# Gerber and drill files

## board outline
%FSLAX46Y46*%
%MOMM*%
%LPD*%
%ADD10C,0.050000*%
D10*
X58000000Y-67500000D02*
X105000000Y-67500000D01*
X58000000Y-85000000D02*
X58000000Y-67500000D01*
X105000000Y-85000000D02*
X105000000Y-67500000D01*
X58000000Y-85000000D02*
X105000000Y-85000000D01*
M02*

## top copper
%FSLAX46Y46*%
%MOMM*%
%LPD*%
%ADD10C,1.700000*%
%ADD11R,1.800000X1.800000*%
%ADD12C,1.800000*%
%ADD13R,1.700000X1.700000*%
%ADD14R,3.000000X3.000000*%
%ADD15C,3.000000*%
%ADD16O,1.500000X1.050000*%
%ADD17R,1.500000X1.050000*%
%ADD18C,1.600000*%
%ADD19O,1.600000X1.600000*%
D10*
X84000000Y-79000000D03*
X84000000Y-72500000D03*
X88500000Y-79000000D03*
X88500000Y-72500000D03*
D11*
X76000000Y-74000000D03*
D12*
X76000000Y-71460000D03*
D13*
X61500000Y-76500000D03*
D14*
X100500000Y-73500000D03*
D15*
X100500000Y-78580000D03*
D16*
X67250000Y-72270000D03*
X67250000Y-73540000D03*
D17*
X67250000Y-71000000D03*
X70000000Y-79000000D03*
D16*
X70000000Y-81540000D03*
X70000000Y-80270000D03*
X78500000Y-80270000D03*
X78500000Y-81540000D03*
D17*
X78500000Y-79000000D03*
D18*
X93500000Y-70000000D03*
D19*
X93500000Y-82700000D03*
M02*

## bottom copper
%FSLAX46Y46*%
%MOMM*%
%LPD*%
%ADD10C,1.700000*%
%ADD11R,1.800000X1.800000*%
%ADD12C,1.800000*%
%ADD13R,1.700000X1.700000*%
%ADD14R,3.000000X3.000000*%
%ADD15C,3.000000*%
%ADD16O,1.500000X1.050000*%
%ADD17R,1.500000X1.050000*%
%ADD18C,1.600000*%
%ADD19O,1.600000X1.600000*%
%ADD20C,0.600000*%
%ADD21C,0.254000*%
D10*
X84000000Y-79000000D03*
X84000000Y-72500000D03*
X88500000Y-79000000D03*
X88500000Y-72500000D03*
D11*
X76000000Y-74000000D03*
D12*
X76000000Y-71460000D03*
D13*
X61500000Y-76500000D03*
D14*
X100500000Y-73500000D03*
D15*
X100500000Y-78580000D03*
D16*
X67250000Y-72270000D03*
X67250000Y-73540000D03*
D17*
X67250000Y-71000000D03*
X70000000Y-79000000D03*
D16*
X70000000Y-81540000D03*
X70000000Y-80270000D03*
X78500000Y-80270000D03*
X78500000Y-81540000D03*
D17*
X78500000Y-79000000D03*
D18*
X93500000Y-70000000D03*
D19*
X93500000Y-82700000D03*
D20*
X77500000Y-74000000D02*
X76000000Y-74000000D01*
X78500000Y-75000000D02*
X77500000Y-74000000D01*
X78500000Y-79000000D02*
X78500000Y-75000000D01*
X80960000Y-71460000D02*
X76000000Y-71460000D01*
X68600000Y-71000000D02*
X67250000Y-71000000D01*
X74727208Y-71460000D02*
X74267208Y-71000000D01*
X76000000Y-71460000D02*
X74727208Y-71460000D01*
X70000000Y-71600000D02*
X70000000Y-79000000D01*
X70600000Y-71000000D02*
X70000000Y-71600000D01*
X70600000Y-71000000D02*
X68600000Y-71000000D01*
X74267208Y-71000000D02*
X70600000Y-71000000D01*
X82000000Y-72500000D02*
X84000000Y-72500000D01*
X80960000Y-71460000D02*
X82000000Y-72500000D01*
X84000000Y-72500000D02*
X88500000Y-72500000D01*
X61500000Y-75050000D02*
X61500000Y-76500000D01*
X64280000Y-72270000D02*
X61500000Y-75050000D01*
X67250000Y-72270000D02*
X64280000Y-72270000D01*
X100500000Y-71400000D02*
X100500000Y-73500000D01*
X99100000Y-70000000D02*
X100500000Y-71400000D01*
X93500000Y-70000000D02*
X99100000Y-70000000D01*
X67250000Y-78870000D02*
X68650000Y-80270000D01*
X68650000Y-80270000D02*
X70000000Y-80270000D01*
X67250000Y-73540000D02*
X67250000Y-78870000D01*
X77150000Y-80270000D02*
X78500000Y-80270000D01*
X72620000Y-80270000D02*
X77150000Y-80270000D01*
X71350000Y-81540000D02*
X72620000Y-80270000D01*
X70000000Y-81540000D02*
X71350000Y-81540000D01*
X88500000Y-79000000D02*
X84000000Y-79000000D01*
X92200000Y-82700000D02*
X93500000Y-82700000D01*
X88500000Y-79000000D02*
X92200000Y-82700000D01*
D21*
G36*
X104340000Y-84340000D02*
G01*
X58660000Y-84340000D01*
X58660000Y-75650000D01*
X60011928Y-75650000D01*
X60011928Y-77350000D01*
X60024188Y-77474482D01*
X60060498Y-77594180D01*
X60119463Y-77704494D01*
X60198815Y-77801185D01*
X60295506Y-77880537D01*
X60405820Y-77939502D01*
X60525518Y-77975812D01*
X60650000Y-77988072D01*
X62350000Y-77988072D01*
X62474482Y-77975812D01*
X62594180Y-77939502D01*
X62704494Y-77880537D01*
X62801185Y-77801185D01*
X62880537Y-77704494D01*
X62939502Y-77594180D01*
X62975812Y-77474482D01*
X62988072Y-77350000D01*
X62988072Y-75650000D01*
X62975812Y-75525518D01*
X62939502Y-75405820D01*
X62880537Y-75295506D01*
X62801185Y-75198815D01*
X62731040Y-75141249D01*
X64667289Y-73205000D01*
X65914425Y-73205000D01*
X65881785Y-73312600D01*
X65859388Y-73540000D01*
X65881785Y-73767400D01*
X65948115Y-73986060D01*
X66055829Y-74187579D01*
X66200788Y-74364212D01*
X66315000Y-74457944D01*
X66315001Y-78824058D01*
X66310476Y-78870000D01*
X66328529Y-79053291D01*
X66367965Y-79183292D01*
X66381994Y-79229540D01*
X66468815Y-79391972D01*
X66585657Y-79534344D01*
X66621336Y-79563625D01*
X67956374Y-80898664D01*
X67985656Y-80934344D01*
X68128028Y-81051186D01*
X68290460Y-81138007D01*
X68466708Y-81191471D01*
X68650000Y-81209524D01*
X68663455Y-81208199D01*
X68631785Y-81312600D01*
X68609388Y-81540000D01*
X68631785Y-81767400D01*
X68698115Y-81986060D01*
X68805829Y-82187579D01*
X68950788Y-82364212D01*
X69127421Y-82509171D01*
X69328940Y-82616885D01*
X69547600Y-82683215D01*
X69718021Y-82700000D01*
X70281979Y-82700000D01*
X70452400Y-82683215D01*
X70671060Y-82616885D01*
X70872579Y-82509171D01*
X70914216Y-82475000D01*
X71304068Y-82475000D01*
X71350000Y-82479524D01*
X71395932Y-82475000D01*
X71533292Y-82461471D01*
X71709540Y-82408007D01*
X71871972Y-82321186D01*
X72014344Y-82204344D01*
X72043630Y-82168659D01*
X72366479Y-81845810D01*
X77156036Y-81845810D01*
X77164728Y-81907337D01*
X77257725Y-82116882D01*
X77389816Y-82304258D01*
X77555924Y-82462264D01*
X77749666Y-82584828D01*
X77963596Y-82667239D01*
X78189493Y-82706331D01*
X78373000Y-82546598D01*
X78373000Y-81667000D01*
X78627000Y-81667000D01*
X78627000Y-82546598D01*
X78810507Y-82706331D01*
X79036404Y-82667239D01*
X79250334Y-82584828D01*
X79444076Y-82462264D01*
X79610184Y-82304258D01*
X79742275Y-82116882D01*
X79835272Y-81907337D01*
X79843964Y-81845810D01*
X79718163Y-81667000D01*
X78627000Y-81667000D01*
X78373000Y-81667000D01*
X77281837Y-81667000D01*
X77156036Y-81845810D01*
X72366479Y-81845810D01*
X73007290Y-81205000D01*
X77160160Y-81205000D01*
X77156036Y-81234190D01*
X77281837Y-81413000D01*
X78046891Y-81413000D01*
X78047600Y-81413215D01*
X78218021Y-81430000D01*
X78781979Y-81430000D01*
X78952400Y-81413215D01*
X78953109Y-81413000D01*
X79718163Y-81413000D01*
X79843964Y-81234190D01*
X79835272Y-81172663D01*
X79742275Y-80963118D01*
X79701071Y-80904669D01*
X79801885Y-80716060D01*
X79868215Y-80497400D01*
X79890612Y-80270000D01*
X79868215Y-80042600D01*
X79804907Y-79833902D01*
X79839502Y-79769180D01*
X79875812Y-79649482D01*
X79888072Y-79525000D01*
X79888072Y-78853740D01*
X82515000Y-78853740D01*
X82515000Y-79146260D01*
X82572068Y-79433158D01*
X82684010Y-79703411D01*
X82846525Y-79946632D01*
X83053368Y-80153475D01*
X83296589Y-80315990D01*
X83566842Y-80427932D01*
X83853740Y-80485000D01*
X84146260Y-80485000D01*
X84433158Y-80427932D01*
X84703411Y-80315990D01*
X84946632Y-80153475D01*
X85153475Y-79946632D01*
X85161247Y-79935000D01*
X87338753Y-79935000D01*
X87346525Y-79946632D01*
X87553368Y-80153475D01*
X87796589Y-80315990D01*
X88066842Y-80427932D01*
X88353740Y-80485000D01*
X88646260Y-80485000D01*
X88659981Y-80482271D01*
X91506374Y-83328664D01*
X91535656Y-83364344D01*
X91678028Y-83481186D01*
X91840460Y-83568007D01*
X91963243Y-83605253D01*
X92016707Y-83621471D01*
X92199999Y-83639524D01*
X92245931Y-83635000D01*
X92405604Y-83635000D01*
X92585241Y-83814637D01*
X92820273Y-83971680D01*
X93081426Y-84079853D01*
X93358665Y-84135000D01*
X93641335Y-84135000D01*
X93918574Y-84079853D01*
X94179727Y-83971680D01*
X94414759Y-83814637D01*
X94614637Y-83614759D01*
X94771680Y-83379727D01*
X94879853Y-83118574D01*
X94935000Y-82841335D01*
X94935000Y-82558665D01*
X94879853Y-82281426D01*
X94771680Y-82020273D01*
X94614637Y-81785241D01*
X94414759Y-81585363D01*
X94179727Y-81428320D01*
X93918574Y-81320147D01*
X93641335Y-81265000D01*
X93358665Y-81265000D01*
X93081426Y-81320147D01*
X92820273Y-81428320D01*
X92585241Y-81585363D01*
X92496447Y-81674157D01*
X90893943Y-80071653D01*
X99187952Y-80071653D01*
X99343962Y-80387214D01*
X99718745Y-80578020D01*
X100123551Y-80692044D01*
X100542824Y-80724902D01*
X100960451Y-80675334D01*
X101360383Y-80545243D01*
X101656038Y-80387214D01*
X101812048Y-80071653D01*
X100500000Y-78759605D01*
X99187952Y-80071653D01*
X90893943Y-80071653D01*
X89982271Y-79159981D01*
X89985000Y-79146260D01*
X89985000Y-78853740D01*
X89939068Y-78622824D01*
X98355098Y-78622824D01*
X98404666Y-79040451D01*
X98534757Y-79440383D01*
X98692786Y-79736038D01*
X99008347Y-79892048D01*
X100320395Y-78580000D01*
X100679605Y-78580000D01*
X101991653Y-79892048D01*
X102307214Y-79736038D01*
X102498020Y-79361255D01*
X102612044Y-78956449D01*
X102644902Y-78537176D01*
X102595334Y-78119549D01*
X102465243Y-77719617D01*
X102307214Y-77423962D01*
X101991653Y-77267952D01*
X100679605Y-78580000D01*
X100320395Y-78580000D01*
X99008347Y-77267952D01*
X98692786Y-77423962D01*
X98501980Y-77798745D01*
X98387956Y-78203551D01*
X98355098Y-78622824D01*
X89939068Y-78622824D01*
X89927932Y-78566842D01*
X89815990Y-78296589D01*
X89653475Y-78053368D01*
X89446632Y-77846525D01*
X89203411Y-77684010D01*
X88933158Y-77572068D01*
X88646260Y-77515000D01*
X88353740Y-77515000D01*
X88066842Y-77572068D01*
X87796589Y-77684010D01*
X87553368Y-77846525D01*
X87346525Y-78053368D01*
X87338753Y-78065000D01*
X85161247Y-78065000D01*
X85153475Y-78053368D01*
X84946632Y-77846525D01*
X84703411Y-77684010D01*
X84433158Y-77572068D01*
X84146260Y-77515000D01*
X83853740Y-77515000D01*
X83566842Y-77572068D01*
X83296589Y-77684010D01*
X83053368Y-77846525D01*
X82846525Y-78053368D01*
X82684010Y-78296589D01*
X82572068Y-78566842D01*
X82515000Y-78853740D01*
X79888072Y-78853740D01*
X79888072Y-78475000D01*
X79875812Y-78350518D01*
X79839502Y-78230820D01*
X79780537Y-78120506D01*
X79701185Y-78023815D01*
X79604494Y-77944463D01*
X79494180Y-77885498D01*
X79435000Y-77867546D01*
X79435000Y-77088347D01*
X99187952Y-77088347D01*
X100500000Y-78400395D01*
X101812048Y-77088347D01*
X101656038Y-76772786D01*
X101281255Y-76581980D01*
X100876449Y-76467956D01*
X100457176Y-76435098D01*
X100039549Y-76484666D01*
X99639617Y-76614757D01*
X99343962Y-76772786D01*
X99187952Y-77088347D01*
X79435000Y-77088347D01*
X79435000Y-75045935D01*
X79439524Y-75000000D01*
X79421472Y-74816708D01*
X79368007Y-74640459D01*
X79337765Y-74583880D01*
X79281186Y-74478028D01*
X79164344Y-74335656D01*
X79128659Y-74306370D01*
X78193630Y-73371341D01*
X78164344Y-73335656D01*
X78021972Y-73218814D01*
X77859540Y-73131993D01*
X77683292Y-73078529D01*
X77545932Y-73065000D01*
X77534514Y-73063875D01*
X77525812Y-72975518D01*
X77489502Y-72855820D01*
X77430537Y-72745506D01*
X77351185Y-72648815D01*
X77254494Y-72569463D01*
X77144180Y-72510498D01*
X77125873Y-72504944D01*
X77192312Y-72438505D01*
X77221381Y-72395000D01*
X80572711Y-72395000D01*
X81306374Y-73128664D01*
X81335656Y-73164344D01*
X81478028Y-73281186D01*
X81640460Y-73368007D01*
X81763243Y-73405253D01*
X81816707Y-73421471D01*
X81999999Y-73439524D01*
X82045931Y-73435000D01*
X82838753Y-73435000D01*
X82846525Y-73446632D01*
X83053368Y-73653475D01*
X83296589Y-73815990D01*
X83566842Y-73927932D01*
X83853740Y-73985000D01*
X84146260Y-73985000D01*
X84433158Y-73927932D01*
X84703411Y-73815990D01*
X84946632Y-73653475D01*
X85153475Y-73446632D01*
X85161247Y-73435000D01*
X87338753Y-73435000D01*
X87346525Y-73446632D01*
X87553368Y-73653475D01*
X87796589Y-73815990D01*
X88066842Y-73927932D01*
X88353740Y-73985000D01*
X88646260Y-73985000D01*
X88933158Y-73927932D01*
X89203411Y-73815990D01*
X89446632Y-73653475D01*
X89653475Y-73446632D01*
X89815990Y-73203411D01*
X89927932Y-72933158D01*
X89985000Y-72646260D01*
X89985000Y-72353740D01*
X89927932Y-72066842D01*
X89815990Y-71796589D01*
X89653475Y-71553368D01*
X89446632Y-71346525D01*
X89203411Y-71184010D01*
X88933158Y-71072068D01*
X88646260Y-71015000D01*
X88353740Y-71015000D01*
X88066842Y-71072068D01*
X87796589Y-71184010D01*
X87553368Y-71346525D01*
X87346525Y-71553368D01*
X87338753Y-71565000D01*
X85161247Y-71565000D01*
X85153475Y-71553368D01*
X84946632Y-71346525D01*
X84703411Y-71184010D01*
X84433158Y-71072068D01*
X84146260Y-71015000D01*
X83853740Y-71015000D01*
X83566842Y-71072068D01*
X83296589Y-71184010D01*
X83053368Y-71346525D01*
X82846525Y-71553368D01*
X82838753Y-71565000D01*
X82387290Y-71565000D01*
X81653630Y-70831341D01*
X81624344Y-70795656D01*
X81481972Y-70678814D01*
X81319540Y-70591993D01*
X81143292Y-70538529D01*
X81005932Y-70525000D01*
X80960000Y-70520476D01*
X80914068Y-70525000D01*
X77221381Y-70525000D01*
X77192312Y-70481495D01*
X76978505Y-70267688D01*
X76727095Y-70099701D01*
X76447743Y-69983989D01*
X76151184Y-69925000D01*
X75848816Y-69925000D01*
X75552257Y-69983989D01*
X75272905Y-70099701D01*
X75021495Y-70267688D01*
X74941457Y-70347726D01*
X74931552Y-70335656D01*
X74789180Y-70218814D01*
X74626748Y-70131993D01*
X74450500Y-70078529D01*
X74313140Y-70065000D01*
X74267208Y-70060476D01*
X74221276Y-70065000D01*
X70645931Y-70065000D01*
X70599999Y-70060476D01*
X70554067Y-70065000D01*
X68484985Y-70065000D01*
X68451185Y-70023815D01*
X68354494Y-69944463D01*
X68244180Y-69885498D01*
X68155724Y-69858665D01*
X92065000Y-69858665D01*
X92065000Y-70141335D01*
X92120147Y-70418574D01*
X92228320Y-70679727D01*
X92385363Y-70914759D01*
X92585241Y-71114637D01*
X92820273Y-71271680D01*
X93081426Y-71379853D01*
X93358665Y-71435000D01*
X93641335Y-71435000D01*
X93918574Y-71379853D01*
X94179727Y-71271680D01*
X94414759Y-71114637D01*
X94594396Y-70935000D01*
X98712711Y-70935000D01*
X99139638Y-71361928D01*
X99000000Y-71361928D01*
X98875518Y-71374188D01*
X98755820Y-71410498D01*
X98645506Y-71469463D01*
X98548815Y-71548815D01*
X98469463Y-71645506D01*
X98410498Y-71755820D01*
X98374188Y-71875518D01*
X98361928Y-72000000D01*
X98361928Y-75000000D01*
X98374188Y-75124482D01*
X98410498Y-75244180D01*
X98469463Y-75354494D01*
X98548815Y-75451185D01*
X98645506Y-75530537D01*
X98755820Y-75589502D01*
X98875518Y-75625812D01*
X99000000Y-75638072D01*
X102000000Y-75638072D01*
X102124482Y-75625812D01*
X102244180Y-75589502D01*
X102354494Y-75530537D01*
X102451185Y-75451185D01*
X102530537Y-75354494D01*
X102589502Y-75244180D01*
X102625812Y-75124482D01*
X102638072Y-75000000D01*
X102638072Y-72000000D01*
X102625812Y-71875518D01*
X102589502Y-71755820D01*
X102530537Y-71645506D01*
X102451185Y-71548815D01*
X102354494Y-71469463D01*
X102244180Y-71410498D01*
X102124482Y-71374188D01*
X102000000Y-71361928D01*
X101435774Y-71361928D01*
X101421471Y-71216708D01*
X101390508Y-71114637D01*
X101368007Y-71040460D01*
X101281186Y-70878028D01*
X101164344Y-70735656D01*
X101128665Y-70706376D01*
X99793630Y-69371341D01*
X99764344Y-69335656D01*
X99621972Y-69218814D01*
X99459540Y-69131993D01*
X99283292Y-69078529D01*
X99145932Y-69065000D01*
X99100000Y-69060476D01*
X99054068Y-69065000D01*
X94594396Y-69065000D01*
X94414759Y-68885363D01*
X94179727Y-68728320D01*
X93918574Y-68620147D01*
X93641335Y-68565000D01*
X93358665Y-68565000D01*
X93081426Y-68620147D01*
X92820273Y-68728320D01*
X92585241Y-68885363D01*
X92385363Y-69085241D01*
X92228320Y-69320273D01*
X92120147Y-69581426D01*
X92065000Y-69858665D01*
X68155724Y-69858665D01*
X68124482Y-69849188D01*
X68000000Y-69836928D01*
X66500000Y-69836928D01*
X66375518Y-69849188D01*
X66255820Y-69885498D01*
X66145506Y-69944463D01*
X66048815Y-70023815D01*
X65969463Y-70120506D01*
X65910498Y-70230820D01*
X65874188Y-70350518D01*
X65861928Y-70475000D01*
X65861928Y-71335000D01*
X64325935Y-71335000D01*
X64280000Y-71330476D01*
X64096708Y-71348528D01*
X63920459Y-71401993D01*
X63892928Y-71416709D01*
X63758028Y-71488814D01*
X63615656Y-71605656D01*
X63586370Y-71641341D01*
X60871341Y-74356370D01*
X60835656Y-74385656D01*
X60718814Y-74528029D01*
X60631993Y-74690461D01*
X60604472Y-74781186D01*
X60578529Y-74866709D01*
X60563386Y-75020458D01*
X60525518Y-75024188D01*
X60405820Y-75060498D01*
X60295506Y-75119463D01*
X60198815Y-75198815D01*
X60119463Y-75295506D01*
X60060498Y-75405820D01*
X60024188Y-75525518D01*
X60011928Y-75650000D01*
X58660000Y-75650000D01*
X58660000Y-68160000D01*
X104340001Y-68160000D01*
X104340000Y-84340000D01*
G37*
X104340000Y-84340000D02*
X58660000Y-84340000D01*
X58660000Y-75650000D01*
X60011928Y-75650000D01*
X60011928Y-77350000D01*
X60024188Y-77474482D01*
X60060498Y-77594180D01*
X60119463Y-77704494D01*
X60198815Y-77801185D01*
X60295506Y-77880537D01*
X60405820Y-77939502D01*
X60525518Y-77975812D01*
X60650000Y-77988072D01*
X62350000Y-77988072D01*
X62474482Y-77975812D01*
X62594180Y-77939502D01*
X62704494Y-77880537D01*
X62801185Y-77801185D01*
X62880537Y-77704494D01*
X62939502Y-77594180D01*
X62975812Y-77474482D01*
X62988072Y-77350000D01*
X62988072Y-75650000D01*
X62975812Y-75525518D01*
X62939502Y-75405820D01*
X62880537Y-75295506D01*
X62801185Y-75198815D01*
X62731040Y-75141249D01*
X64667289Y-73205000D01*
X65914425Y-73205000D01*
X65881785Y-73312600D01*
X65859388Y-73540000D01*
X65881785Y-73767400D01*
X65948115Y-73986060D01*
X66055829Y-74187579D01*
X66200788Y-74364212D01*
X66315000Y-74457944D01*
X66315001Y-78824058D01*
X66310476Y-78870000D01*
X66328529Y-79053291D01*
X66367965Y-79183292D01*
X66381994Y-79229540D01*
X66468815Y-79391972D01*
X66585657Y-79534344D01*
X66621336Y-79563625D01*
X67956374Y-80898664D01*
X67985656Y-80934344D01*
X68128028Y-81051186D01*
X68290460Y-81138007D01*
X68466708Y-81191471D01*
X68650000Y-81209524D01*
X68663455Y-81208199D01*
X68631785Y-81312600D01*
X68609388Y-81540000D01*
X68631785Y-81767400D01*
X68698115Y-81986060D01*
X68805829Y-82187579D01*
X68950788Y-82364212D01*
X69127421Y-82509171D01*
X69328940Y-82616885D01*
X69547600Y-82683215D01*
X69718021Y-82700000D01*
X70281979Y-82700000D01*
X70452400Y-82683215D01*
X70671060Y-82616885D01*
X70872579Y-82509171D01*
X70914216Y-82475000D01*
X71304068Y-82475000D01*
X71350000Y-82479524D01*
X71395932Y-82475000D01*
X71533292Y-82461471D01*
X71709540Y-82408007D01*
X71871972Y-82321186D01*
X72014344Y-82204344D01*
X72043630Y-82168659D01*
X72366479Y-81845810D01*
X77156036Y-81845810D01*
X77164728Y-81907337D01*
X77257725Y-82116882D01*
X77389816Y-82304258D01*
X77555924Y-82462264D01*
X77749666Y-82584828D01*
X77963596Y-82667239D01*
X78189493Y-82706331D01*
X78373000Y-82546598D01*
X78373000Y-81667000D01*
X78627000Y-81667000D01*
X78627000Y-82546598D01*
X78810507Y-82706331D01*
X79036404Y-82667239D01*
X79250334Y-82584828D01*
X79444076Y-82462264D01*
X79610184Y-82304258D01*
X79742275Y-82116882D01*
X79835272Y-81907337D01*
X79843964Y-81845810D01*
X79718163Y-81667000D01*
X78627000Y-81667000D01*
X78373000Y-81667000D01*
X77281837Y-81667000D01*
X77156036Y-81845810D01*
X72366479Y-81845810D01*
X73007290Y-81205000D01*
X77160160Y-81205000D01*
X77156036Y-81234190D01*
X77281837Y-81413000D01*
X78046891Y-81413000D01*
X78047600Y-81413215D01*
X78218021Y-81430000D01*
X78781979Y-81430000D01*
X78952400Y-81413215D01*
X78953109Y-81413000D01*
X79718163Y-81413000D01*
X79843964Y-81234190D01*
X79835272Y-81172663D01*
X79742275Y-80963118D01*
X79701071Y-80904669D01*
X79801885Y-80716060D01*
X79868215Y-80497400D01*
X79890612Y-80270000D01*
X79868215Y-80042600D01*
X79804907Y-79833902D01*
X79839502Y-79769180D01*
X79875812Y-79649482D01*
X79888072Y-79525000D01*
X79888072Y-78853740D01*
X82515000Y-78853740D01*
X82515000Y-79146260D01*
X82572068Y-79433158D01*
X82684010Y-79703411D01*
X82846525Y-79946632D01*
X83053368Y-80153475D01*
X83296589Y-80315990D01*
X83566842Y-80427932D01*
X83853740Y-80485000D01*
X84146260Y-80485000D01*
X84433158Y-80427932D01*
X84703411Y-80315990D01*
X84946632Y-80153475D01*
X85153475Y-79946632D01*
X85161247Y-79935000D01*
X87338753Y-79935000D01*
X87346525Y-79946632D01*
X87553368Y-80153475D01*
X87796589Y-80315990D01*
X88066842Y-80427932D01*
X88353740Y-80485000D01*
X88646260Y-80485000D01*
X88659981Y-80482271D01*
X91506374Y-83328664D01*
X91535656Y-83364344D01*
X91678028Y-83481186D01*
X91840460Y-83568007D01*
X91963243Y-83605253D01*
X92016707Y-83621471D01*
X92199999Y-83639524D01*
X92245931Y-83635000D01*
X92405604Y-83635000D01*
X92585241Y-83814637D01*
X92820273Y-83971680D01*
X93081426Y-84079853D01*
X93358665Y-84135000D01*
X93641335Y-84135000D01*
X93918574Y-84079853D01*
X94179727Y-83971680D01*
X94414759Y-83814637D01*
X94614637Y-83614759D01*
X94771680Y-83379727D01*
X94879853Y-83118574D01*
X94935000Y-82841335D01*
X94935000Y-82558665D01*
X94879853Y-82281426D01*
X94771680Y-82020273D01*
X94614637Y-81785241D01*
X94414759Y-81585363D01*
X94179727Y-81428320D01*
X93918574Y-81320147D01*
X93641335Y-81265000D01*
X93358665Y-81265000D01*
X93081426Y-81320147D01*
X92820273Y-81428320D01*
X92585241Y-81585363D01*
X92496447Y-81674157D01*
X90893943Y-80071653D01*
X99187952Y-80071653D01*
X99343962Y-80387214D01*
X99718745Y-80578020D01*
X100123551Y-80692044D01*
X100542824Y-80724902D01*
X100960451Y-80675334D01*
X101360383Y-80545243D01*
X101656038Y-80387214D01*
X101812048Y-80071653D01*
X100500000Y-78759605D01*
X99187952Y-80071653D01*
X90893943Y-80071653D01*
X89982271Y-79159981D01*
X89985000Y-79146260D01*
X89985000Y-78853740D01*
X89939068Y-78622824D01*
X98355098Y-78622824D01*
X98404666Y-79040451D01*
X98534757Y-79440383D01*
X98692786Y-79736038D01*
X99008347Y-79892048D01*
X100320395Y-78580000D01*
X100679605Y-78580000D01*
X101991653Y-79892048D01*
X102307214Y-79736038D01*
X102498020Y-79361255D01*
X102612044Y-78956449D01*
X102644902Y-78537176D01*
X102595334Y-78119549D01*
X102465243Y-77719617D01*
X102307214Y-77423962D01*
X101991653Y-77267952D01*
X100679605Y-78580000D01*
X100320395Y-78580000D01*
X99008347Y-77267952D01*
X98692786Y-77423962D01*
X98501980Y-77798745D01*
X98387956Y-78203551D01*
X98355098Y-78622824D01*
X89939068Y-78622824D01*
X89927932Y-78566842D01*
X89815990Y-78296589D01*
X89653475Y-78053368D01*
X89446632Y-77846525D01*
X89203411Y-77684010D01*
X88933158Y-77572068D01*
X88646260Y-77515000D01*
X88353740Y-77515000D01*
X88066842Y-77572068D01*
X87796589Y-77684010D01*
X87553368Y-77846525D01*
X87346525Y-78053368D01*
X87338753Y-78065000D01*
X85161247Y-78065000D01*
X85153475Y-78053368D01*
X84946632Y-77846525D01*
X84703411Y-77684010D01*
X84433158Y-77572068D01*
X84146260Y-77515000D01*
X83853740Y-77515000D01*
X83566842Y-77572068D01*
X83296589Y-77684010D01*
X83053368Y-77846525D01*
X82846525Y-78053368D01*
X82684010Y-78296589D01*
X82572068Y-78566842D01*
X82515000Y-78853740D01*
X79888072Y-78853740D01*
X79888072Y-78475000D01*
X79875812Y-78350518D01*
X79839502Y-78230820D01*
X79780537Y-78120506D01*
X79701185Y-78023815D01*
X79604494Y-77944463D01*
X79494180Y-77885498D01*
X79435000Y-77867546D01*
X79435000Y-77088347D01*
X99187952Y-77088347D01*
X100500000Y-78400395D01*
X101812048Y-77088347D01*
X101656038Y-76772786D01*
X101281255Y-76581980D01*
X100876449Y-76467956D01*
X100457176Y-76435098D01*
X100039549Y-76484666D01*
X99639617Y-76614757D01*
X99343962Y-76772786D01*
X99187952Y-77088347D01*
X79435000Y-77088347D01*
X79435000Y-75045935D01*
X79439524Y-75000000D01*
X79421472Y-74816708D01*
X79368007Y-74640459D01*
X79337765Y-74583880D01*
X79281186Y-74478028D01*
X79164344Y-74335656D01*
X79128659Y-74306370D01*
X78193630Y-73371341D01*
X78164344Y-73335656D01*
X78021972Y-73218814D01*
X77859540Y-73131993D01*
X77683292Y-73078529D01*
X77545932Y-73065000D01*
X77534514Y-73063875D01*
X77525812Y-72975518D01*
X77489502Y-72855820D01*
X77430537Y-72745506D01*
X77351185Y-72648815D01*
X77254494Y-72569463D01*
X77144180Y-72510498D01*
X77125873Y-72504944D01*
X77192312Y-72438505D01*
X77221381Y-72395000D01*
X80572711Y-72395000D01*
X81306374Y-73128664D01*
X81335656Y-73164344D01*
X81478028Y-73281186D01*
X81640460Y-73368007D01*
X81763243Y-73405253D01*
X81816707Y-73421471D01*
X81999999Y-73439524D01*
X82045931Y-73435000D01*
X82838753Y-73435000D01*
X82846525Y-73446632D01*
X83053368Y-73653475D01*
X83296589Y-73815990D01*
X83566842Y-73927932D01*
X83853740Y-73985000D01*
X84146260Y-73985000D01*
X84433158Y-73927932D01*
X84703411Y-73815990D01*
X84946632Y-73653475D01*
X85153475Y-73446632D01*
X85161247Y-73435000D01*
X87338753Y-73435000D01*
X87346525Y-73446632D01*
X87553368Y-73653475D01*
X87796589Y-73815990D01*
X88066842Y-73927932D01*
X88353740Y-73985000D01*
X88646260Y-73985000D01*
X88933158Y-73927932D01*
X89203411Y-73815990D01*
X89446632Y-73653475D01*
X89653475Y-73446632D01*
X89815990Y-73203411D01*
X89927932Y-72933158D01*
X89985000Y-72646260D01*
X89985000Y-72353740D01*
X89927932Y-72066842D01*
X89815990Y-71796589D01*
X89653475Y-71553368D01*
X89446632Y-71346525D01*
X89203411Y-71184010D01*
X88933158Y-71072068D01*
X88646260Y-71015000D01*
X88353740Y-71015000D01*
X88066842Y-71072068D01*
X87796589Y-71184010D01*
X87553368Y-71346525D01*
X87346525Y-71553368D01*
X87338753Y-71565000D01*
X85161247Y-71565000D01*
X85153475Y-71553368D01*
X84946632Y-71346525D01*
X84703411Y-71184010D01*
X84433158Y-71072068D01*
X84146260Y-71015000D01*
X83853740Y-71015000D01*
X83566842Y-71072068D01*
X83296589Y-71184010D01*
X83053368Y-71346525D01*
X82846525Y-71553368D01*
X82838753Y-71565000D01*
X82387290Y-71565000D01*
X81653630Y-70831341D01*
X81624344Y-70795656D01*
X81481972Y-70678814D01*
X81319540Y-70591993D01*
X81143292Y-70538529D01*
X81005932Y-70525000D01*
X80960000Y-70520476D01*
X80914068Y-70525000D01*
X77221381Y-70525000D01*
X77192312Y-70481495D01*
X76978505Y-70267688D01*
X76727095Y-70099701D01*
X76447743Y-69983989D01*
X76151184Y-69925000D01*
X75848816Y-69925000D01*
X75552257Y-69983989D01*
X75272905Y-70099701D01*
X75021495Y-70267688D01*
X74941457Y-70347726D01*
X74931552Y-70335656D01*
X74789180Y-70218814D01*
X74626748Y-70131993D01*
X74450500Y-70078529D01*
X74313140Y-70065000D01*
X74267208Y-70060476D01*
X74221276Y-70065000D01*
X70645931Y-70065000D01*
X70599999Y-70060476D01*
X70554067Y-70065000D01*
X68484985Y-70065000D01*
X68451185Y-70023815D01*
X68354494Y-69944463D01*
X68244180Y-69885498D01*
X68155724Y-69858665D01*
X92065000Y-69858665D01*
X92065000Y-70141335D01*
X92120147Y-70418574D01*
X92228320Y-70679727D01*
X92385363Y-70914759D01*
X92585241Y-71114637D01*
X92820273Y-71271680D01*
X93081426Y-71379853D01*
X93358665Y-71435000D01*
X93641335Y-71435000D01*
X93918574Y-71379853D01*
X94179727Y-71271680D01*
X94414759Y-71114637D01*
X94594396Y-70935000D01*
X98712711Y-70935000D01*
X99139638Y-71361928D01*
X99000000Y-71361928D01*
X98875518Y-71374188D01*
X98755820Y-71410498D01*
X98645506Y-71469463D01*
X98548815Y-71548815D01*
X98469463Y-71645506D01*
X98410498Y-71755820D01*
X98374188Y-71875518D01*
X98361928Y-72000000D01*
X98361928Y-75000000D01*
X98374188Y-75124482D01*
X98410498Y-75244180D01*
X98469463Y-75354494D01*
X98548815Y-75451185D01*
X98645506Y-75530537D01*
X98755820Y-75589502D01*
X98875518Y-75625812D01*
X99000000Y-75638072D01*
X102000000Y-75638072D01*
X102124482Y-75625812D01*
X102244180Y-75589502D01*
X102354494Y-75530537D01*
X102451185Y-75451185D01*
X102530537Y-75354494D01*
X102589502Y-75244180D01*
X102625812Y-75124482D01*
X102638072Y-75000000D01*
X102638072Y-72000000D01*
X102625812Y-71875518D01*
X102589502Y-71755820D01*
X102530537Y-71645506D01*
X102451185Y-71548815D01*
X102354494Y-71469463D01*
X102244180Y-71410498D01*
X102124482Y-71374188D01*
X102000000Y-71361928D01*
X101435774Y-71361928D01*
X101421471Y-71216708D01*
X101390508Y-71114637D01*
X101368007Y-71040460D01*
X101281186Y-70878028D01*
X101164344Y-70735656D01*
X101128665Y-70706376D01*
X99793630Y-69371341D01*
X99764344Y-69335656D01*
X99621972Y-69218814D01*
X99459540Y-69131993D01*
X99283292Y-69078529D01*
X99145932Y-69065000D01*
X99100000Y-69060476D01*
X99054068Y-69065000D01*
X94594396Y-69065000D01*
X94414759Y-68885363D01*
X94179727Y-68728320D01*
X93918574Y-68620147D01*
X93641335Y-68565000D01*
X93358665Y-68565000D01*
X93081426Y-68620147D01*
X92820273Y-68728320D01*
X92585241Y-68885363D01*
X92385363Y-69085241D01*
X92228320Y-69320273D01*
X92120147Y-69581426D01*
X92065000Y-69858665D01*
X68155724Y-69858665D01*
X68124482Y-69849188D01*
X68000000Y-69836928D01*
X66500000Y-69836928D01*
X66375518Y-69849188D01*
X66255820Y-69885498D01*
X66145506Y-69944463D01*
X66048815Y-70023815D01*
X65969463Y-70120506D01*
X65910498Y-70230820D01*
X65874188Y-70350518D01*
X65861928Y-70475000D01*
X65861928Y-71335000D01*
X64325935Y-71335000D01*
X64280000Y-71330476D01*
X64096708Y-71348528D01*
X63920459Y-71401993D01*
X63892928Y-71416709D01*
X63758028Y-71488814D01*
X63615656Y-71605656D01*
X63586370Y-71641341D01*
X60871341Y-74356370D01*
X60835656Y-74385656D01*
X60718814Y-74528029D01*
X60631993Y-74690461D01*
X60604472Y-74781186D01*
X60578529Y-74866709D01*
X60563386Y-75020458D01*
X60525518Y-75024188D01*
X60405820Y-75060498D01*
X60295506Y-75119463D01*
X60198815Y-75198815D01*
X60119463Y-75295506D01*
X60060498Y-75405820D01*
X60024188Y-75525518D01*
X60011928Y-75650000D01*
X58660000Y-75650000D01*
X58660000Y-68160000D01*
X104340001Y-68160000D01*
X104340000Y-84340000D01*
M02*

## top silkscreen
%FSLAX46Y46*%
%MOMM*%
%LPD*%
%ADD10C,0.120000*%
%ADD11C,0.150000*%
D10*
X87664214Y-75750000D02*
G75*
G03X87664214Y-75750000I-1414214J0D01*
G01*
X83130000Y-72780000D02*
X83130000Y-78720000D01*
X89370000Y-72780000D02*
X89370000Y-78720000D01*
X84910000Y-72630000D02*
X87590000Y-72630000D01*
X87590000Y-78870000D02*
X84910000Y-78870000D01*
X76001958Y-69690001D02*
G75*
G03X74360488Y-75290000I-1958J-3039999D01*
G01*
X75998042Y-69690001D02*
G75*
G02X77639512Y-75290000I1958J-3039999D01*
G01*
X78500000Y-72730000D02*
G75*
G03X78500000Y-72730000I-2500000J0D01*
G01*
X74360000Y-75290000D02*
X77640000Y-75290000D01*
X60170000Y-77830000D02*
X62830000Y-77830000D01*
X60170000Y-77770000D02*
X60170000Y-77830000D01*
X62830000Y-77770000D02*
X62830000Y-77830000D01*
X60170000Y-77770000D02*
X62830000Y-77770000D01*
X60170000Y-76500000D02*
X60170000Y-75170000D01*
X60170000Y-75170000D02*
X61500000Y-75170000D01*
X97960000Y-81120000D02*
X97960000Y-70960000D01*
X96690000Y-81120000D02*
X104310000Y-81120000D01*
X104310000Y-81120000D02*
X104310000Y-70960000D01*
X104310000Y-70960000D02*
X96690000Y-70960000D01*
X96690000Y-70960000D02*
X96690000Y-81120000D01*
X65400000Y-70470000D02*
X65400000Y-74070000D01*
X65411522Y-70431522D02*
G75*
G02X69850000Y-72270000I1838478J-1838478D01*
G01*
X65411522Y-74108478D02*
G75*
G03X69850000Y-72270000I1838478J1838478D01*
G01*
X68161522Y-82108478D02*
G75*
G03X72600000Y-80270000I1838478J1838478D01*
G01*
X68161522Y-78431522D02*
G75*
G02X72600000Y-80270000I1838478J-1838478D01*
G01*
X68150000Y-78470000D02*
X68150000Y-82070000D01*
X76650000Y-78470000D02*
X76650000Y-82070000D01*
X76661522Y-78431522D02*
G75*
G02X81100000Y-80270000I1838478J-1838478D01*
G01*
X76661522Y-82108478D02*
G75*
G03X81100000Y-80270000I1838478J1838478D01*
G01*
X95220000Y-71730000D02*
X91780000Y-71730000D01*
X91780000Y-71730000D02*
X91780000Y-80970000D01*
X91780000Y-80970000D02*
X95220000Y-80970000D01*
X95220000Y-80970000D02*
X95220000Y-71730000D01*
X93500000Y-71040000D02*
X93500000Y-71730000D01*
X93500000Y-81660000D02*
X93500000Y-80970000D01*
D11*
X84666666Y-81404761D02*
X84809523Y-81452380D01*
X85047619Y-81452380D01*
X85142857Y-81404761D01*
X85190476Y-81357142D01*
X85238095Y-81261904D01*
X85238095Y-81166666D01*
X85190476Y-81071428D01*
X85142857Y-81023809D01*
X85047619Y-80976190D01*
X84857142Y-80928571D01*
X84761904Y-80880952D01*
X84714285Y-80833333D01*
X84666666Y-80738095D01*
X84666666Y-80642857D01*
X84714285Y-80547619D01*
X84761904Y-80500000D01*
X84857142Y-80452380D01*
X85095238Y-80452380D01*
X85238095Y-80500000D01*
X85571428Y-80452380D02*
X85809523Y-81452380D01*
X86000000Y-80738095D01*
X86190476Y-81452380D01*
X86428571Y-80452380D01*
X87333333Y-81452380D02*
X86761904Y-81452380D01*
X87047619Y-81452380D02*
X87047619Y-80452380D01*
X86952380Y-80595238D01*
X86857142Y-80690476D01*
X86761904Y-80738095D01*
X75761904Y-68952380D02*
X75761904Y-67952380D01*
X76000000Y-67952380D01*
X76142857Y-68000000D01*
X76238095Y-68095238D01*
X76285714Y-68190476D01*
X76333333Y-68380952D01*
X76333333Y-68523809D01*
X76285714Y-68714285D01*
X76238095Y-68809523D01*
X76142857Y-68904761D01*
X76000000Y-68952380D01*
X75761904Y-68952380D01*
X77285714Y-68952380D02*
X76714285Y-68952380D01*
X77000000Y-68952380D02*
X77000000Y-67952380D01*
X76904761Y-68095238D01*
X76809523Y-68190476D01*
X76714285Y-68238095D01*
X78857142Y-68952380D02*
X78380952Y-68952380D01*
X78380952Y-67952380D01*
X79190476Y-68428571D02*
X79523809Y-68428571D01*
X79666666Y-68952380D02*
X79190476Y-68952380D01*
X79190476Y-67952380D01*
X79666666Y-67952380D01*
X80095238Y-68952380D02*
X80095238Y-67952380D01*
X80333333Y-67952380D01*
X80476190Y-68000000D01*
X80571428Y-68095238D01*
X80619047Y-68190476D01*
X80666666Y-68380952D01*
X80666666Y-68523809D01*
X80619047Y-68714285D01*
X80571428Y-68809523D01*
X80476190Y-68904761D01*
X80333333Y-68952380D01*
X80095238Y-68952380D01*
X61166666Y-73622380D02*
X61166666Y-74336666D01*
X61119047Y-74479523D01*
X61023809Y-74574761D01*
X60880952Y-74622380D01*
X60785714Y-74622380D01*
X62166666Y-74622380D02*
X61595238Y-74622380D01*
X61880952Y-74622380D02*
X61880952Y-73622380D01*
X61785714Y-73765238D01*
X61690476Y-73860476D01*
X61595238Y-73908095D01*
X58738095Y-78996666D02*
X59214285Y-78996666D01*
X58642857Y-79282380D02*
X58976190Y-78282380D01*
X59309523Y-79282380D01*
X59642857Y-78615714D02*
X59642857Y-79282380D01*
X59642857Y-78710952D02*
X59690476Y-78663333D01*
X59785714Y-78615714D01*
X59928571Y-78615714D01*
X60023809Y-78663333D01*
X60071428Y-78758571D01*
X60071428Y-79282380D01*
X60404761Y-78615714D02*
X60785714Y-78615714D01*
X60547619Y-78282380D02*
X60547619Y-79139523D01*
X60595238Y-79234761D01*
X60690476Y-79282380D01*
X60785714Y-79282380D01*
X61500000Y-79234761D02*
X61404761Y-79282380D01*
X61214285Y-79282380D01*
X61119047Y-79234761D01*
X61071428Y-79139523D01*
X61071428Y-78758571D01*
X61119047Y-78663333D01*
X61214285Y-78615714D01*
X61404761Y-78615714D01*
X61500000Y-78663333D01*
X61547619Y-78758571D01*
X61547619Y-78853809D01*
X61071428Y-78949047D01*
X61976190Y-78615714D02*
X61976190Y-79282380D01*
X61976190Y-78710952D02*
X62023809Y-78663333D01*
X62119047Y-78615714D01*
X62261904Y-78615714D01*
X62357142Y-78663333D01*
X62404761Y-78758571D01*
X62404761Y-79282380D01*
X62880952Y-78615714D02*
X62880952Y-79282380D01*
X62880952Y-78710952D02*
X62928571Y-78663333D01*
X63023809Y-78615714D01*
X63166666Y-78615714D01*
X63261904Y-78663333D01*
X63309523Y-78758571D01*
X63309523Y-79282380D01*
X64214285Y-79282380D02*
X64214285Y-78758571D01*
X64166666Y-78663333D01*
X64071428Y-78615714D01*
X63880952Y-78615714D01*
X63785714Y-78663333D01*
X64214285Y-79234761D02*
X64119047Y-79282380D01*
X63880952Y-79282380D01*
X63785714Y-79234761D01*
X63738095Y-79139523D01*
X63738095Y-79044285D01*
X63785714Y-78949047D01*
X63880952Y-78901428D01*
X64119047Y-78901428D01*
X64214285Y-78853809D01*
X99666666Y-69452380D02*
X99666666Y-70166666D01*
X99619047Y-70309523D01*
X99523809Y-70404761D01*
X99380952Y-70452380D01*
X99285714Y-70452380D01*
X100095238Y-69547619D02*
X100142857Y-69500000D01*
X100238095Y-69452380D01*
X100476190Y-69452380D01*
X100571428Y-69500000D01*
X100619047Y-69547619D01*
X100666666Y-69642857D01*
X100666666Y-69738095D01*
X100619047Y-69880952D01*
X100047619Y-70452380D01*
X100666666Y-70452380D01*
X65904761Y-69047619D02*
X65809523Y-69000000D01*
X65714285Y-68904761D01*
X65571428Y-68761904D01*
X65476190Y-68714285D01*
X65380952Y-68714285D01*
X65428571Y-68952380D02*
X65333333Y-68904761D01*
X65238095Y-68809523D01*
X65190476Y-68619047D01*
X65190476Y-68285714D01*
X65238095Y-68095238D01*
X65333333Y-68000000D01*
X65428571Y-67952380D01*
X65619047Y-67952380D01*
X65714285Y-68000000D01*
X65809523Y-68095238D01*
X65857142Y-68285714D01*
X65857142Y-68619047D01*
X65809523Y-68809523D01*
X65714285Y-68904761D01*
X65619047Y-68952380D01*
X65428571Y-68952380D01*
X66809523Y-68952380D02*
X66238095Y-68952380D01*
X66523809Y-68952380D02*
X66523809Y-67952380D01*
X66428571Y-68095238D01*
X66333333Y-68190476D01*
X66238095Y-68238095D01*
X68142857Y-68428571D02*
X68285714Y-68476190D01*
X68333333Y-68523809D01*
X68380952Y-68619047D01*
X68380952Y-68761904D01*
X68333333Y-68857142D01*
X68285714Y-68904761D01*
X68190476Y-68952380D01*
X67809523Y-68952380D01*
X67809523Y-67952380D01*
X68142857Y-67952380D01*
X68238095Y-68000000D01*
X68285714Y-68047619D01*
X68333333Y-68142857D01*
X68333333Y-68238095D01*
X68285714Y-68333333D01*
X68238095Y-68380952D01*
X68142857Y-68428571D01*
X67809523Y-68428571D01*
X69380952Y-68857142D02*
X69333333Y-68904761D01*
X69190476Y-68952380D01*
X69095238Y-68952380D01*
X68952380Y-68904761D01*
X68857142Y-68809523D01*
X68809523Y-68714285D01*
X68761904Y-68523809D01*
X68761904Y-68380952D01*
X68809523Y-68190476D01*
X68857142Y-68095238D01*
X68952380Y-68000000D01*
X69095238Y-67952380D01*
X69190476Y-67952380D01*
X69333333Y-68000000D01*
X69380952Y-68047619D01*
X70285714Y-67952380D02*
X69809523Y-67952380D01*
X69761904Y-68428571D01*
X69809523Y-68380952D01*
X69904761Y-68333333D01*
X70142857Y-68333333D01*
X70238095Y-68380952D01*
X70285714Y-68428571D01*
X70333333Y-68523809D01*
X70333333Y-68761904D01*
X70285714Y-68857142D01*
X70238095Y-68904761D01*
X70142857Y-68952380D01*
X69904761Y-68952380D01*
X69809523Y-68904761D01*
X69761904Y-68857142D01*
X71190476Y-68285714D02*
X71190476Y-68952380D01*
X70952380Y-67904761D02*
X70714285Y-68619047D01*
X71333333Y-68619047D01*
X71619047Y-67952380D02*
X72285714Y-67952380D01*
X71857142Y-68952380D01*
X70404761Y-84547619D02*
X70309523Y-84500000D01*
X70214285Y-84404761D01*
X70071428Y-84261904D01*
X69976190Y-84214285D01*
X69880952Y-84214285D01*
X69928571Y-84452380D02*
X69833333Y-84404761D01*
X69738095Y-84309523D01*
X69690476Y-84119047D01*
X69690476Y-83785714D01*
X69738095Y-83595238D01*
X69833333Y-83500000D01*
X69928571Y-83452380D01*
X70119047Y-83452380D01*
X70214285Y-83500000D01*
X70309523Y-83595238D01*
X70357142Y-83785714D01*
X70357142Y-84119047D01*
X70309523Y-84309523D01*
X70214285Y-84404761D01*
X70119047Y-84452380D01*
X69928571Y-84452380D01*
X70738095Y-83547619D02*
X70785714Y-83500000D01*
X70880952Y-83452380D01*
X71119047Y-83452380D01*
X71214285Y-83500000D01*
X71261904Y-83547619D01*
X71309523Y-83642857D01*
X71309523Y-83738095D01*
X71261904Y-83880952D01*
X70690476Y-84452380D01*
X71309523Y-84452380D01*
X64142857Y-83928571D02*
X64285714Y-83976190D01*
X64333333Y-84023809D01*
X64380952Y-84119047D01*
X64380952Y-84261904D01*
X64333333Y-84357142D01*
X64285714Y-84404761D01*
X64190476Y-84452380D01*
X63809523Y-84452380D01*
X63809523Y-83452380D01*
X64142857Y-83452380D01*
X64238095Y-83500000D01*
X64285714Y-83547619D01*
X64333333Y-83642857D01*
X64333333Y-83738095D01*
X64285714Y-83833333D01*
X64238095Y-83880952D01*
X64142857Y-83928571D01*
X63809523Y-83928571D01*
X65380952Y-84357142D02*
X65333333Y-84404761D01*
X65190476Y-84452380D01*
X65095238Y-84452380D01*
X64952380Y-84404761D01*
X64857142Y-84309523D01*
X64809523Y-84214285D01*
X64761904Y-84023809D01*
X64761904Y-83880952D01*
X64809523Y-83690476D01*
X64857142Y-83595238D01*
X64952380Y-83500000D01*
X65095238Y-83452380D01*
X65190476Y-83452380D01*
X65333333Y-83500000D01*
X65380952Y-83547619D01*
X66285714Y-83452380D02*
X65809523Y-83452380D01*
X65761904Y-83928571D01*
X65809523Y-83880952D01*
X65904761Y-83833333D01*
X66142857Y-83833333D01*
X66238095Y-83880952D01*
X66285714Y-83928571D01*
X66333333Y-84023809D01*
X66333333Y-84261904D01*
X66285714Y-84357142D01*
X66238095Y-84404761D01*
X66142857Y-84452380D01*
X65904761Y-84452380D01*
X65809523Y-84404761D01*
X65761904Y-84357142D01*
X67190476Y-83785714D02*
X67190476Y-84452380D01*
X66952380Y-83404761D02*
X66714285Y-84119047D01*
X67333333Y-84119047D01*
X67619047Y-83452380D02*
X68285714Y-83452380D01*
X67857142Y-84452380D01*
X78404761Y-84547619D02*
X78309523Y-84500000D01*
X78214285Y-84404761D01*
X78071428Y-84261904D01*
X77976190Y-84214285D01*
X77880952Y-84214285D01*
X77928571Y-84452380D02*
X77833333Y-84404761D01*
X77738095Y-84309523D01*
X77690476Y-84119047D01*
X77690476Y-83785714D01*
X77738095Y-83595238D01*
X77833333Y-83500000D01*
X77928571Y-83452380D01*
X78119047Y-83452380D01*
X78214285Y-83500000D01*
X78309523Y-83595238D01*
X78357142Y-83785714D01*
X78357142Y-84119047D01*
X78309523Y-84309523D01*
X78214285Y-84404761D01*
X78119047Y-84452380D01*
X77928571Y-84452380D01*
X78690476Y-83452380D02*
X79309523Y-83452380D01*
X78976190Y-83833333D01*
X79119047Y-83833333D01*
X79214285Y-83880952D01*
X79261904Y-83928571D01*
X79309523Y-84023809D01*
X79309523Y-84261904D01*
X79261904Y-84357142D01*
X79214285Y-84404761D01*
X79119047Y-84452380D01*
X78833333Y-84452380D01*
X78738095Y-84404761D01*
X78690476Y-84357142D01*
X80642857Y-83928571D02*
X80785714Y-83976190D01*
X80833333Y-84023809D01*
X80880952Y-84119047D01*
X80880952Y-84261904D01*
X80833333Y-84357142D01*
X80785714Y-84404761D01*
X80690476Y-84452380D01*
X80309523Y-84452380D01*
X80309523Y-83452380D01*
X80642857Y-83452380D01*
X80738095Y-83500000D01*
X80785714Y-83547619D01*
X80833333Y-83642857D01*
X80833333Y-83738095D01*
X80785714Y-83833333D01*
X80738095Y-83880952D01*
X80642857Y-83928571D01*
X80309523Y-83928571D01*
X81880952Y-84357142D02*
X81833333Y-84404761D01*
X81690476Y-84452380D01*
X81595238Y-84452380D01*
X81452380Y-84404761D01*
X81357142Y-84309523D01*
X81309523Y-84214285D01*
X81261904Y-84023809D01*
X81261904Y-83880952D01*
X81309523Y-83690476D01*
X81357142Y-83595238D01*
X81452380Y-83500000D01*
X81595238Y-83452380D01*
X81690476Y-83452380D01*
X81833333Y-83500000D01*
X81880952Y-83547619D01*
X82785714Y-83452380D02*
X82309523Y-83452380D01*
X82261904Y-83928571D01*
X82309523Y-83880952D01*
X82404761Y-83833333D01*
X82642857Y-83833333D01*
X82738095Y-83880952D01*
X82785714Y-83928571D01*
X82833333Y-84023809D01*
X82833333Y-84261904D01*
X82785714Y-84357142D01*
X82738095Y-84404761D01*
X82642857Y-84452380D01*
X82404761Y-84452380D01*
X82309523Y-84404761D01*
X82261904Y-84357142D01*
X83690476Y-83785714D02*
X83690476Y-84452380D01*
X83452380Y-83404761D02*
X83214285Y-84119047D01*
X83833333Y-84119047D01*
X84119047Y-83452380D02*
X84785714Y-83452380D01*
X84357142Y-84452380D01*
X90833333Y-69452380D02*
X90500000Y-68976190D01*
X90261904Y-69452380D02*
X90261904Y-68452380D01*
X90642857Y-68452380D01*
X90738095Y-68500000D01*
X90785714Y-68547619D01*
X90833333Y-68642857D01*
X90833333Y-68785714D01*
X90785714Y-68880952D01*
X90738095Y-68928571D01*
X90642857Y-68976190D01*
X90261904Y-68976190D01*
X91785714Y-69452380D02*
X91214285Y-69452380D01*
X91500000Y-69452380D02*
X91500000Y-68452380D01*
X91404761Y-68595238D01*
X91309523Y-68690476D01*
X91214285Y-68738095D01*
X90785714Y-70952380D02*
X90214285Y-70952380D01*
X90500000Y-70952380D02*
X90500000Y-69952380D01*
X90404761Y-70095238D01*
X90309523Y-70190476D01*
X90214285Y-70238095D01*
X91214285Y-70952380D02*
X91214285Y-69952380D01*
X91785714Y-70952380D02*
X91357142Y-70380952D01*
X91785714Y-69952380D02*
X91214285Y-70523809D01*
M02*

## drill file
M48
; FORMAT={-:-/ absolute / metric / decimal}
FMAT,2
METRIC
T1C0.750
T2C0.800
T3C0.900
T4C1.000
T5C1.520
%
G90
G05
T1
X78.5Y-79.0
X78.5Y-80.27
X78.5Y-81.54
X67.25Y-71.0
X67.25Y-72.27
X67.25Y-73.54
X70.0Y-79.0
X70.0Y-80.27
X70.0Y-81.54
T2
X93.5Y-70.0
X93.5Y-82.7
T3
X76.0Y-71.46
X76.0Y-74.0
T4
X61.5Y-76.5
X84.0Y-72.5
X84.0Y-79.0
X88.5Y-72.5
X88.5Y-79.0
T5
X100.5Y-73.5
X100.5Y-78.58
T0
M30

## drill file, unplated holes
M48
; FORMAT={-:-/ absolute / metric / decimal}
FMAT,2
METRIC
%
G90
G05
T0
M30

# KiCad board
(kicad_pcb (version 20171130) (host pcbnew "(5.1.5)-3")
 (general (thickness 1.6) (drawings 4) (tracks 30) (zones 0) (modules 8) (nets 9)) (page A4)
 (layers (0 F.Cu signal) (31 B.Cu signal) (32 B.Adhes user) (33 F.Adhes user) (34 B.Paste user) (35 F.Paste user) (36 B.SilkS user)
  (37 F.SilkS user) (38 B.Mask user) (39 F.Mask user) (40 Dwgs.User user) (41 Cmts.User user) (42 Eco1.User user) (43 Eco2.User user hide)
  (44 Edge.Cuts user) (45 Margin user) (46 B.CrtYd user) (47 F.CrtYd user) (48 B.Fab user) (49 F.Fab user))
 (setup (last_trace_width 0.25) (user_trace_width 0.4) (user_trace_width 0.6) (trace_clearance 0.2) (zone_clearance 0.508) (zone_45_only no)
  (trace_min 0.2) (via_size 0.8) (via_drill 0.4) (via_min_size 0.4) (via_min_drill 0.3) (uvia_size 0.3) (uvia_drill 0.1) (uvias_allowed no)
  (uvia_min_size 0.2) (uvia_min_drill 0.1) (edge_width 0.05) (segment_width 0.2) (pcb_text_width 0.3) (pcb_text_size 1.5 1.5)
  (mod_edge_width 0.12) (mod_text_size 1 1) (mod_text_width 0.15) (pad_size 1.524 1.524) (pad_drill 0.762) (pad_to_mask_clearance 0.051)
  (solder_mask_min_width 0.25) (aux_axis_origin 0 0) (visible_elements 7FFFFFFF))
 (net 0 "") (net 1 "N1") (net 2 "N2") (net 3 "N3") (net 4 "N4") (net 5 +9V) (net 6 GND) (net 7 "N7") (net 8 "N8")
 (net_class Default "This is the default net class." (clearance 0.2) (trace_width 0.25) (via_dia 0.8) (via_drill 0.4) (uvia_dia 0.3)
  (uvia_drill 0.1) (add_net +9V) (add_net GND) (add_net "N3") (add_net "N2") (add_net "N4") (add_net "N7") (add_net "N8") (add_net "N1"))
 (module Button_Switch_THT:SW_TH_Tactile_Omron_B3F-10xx (layer F.Cu) (at 88.5 72.5 270)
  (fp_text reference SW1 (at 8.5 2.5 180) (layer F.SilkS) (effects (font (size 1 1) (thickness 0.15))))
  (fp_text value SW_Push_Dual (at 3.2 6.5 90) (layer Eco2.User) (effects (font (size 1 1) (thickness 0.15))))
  (fp_circle (center 3.25 2.25) (end 4.25 3.25) (layer F.SilkS) (width 0.12))
  (fp_line (start 0.28 5.37) (end 6.22 5.37) (layer F.SilkS) (width 0.12))
  (fp_line (start 0.28 -0.87) (end 6.22 -0.87) (layer F.SilkS) (width 0.12))
  (fp_line (start 0.13 3.59) (end 0.13 0.91) (layer F.SilkS) (width 0.12))
  (fp_line (start 6.37 0.91) (end 6.37 3.59) (layer F.SilkS) (width 0.12))
  (pad 4 thru_hole circle (at 6.5 4.5 270) (size 1.7 1.7) (drill 1) (layers *.Cu *.Mask) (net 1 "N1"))
  (pad 3 thru_hole circle (at 0 4.5 270) (size 1.7 1.7) (drill 1) (layers *.Cu *.Mask) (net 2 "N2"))
  (pad 2 thru_hole circle (at 6.5 0 270) (size 1.7 1.7) (drill 1) (layers *.Cu *.Mask) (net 1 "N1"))
  (pad 1 thru_hole circle (at 0 0 270) (size 1.7 1.7) (drill 1) (layers *.Cu *.Mask) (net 2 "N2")))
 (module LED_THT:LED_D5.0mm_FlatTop (layer F.Cu) (at 76 74 90)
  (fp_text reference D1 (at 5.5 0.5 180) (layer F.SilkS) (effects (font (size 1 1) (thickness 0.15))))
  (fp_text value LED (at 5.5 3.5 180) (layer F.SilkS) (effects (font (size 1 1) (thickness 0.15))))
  (fp_arc (start 1.27 0) (end -1.29 -1.639512) (angle 147.4) (layer F.SilkS) (width 0.12))
  (fp_arc (start 1.27 0) (end -1.29 1.639512) (angle -147.4) (layer F.SilkS) (width 0.12))
  (fp_circle (center 1.27 0) (end 3.77 0) (layer F.SilkS) (width 0.12))
  (fp_line (start -1.29 -1.64) (end -1.29 1.64) (layer F.SilkS) (width 0.12))
  (pad 1 thru_hole rect (at 0 0 90) (size 1.8 1.8) (drill 0.9) (layers *.Cu *.Mask) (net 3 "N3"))
  (pad 2 thru_hole circle (at 2.54 0 90) (size 1.8 1.8) (drill 0.9) (layers *.Cu *.Mask) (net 2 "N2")))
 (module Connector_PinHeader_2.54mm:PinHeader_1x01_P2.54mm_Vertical (layer F.Cu) (at 61.5 76.5)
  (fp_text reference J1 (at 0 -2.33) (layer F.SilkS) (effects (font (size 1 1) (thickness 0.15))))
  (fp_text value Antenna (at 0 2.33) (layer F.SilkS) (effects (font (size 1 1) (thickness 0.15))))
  (fp_line (start -1.33 1.33) (end 1.33 1.33) (layer F.SilkS) (width 0.12))
  (fp_line (start -1.33 1.27) (end -1.33 1.33) (layer F.SilkS) (width 0.12))
  (fp_line (start 1.33 1.27) (end 1.33 1.33) (layer F.SilkS) (width 0.12))
  (fp_line (start -1.33 1.27) (end 1.33 1.27) (layer F.SilkS) (width 0.12))
  (fp_line (start -1.33 0) (end -1.33 -1.33) (layer F.SilkS) (width 0.12))
  (fp_line (start -1.33 -1.33) (end 0 -1.33) (layer F.SilkS) (width 0.12))
  (pad 1 thru_hole rect (at 0 0) (size 1.7 1.7) (drill 1) (layers *.Cu *.Mask) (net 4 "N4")))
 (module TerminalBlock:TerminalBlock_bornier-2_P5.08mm (layer F.Cu) (at 100.5 73.5 270)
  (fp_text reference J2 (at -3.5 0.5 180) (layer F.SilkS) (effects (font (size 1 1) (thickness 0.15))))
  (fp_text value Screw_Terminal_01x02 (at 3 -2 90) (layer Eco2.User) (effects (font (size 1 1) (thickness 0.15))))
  (fp_line (start 7.62 2.54) (end -2.54 2.54) (layer F.SilkS) (width 0.12))
  (fp_line (start 7.62 3.81) (end 7.62 -3.81) (layer F.SilkS) (width 0.12))
  (fp_line (start 7.62 -3.81) (end -2.54 -3.81) (layer F.SilkS) (width 0.12))
  (fp_line (start -2.54 -3.81) (end -2.54 3.81) (layer F.SilkS) (width 0.12))
  (fp_line (start -2.54 3.81) (end 7.62 3.81) (layer F.SilkS) (width 0.12))
  (pad 1 thru_hole rect (at 0 0 270) (size 3 3) (drill 1.52) (layers *.Cu *.Mask) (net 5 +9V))
  (pad 2 thru_hole circle (at 5.08 0 270) (size 3 3) (drill 1.52) (layers *.Cu *.Mask) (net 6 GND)))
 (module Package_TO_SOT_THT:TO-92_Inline (layer F.Cu) (at 67.25 71 270)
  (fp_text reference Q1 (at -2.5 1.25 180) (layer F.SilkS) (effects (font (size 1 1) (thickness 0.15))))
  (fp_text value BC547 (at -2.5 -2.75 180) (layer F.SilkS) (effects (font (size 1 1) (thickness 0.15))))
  (fp_line (start -0.53 1.85) (end 3.07 1.85) (layer F.SilkS) (width 0.12))
  (fp_arc (start 1.27 0) (end 1.27 -2.6) (angle -135) (layer F.SilkS) (width 0.12))
  (fp_arc (start 1.27 0) (end 1.27 -2.6) (angle 135) (layer F.SilkS) (width 0.12))
  (pad 2 thru_hole oval (at 1.27 0 270) (size 1.05 1.5) (drill 0.75) (layers *.Cu *.Mask) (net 4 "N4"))
  (pad 3 thru_hole oval (at 2.54 0 270) (size 1.05 1.5) (drill 0.75) (layers *.Cu *.Mask) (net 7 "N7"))
  (pad 1 thru_hole rect (at 0 0 270) (size 1.05 1.5) (drill 0.75) (layers *.Cu *.Mask) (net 2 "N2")))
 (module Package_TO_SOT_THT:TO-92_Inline (layer F.Cu) (at 70 79 270)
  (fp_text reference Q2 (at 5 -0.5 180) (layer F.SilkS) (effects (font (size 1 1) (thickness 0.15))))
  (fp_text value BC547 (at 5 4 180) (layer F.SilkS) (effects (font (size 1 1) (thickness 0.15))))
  (fp_arc (start 1.27 0) (end 1.27 -2.6) (angle 135) (layer F.SilkS) (width 0.12))
  (fp_arc (start 1.27 0) (end 1.27 -2.6) (angle -135) (layer F.SilkS) (width 0.12))
  (fp_line (start -0.53 1.85) (end 3.07 1.85) (layer F.SilkS) (width 0.12))
  (pad 1 thru_hole rect (at 0 0 270) (size 1.05 1.5) (drill 0.75) (layers *.Cu *.Mask) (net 2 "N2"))
  (pad 3 thru_hole oval (at 2.54 0 270) (size 1.05 1.5) (drill 0.75) (layers *.Cu *.Mask) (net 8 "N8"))
  (pad 2 thru_hole oval (at 1.27 0 270) (size 1.05 1.5) (drill 0.75) (layers *.Cu *.Mask) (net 7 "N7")))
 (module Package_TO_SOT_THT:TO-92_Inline (layer F.Cu) (at 78.5 79 270)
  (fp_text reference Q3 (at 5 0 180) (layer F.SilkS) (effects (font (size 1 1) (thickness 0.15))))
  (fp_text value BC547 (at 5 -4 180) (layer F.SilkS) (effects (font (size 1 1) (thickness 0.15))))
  (fp_line (start -0.53 1.85) (end 3.07 1.85) (layer F.SilkS) (width 0.12))
  (fp_arc (start 1.27 0) (end 1.27 -2.6) (angle -135) (layer F.SilkS) (width 0.12))
  (fp_arc (start 1.27 0) (end 1.27 -2.6) (angle 135) (layer F.SilkS) (width 0.12))
  (pad 2 thru_hole oval (at 1.27 0 270) (size 1.05 1.5) (drill 0.75) (layers *.Cu *.Mask) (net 8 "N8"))
  (pad 3 thru_hole oval (at 2.54 0 270) (size 1.05 1.5) (drill 0.75) (layers *.Cu *.Mask) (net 6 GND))
  (pad 1 thru_hole rect (at 0 0 270) (size 1.05 1.5) (drill 0.75) (layers *.Cu *.Mask) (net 3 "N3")))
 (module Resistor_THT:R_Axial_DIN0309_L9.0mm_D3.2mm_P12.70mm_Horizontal (layer F.Cu) (at 93.5 70 270)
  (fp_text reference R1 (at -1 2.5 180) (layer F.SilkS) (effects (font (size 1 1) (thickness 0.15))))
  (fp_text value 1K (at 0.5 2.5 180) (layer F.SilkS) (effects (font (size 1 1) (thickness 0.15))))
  (fp_line (start 1.73 -1.72) (end 1.73 1.72) (layer F.SilkS) (width 0.12))
  (fp_line (start 1.73 1.72) (end 10.97 1.72) (layer F.SilkS) (width 0.12))
  (fp_line (start 10.97 1.72) (end 10.97 -1.72) (layer F.SilkS) (width 0.12))
  (fp_line (start 10.97 -1.72) (end 1.73 -1.72) (layer F.SilkS) (width 0.12))
  (fp_line (start 1.04 0) (end 1.73 0) (layer F.SilkS) (width 0.12))
  (fp_line (start 11.66 0) (end 10.97 0) (layer F.SilkS) (width 0.12))
  (pad 1 thru_hole circle (at 0 0 270) (size 1.6 1.6) (drill 0.8) (layers *.Cu *.Mask) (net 5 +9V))
  (pad 2 thru_hole oval (at 12.7 0 270) (size 1.6 1.6) (drill 0.8) (layers *.Cu *.Mask) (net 1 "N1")))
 (gr_line (start 58 67.5) (end 105 67.5) (layer Edge.Cuts) (width 0.05))
 (gr_line (start 58 85) (end 58 67.5) (layer Edge.Cuts) (width 0.05))
 (gr_line (start 105 85) (end 105 67.5) (layer Edge.Cuts) (width 0.05))
 (gr_line (start 58 85) (end 105 85) (layer Edge.Cuts) (width 0.05))
 (segment (start 77.5 74) (end 76 74) (width 0.6) (layer B.Cu) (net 3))
 (segment (start 78.5 75) (end 77.5 74) (width 0.6) (layer B.Cu) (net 3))
 (segment (start 78.5 79) (end 78.5 75) (width 0.6) (layer B.Cu) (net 3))
 (segment (start 80.96 71.46) (end 76 71.46) (width 0.6) (layer B.Cu) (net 2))
 (segment (start 68.6 71) (end 67.25 71) (width 0.6) (layer B.Cu) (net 2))
 (segment (start 74.727208 71.46) (end 74.267208 71) (width 0.6) (layer B.Cu) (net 2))
 (segment (start 76 71.46) (end 74.727208 71.46) (width 0.6) (layer B.Cu) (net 2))
 (segment (start 70 71.6) (end 70 79) (width 0.6) (layer B.Cu) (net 2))
 (segment (start 70.6 71) (end 70 71.6) (width 0.6) (layer B.Cu) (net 2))
 (segment (start 70.6 71) (end 68.6 71) (width 0.6) (layer B.Cu) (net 2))
 (segment (start 74.267208 71) (end 70.6 71) (width 0.6) (layer B.Cu) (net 2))
 (segment (start 82 72.5) (end 84 72.5) (width 0.6) (layer B.Cu) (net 2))
 (segment (start 80.96 71.46) (end 82 72.5) (width 0.6) (layer B.Cu) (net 2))
 (segment (start 84 72.5) (end 88.5 72.5) (width 0.6) (layer B.Cu) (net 2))
 (segment (start 61.5 75.05) (end 61.5 76.5) (width 0.6) (layer B.Cu) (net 4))
 (segment (start 64.28 72.27) (end 61.5 75.05) (width 0.6) (layer B.Cu) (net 4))
 (segment (start 67.25 72.27) (end 64.28 72.27) (width 0.6) (layer B.Cu) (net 4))
 (segment (start 100.5 71.4) (end 100.5 73.5) (width 0.6) (layer B.Cu) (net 5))
 (segment (start 99.1 70) (end 100.5 71.4) (width 0.6) (layer B.Cu) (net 5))
 (segment (start 93.5 70) (end 99.1 70) (width 0.6) (layer B.Cu) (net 5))
 (segment (start 67.25 78.87) (end 68.65 80.27) (width 0.6) (layer B.Cu) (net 7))
 (segment (start 68.65 80.27) (end 70 80.27) (width 0.6) (layer B.Cu) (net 7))
 (segment (start 67.25 73.54) (end 67.25 78.87) (width 0.6) (layer B.Cu) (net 7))
 (segment (start 77.15 80.27) (end 78.5 80.27) (width 0.6) (layer B.Cu) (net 8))
 (segment (start 72.62 80.27) (end 77.15 80.27) (width 0.6) (layer B.Cu) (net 8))
 (segment (start 71.35 81.54) (end 72.62 80.27) (width 0.6) (layer B.Cu) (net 8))
 (segment (start 70 81.54) (end 71.35 81.54) (width 0.6) (layer B.Cu) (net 8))
 (segment (start 88.5 79) (end 84 79) (width 0.6) (layer B.Cu) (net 1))
 (segment (start 92.2 82.7) (end 93.5 82.7) (width 0.6) (layer B.Cu) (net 1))
 (segment (start 88.5 79) (end 92.2 82.7) (width 0.6) (layer B.Cu) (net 1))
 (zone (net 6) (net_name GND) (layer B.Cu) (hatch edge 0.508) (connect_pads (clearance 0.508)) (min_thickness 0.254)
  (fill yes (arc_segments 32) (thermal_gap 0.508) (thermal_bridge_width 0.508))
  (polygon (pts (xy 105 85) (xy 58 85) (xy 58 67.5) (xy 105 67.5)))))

